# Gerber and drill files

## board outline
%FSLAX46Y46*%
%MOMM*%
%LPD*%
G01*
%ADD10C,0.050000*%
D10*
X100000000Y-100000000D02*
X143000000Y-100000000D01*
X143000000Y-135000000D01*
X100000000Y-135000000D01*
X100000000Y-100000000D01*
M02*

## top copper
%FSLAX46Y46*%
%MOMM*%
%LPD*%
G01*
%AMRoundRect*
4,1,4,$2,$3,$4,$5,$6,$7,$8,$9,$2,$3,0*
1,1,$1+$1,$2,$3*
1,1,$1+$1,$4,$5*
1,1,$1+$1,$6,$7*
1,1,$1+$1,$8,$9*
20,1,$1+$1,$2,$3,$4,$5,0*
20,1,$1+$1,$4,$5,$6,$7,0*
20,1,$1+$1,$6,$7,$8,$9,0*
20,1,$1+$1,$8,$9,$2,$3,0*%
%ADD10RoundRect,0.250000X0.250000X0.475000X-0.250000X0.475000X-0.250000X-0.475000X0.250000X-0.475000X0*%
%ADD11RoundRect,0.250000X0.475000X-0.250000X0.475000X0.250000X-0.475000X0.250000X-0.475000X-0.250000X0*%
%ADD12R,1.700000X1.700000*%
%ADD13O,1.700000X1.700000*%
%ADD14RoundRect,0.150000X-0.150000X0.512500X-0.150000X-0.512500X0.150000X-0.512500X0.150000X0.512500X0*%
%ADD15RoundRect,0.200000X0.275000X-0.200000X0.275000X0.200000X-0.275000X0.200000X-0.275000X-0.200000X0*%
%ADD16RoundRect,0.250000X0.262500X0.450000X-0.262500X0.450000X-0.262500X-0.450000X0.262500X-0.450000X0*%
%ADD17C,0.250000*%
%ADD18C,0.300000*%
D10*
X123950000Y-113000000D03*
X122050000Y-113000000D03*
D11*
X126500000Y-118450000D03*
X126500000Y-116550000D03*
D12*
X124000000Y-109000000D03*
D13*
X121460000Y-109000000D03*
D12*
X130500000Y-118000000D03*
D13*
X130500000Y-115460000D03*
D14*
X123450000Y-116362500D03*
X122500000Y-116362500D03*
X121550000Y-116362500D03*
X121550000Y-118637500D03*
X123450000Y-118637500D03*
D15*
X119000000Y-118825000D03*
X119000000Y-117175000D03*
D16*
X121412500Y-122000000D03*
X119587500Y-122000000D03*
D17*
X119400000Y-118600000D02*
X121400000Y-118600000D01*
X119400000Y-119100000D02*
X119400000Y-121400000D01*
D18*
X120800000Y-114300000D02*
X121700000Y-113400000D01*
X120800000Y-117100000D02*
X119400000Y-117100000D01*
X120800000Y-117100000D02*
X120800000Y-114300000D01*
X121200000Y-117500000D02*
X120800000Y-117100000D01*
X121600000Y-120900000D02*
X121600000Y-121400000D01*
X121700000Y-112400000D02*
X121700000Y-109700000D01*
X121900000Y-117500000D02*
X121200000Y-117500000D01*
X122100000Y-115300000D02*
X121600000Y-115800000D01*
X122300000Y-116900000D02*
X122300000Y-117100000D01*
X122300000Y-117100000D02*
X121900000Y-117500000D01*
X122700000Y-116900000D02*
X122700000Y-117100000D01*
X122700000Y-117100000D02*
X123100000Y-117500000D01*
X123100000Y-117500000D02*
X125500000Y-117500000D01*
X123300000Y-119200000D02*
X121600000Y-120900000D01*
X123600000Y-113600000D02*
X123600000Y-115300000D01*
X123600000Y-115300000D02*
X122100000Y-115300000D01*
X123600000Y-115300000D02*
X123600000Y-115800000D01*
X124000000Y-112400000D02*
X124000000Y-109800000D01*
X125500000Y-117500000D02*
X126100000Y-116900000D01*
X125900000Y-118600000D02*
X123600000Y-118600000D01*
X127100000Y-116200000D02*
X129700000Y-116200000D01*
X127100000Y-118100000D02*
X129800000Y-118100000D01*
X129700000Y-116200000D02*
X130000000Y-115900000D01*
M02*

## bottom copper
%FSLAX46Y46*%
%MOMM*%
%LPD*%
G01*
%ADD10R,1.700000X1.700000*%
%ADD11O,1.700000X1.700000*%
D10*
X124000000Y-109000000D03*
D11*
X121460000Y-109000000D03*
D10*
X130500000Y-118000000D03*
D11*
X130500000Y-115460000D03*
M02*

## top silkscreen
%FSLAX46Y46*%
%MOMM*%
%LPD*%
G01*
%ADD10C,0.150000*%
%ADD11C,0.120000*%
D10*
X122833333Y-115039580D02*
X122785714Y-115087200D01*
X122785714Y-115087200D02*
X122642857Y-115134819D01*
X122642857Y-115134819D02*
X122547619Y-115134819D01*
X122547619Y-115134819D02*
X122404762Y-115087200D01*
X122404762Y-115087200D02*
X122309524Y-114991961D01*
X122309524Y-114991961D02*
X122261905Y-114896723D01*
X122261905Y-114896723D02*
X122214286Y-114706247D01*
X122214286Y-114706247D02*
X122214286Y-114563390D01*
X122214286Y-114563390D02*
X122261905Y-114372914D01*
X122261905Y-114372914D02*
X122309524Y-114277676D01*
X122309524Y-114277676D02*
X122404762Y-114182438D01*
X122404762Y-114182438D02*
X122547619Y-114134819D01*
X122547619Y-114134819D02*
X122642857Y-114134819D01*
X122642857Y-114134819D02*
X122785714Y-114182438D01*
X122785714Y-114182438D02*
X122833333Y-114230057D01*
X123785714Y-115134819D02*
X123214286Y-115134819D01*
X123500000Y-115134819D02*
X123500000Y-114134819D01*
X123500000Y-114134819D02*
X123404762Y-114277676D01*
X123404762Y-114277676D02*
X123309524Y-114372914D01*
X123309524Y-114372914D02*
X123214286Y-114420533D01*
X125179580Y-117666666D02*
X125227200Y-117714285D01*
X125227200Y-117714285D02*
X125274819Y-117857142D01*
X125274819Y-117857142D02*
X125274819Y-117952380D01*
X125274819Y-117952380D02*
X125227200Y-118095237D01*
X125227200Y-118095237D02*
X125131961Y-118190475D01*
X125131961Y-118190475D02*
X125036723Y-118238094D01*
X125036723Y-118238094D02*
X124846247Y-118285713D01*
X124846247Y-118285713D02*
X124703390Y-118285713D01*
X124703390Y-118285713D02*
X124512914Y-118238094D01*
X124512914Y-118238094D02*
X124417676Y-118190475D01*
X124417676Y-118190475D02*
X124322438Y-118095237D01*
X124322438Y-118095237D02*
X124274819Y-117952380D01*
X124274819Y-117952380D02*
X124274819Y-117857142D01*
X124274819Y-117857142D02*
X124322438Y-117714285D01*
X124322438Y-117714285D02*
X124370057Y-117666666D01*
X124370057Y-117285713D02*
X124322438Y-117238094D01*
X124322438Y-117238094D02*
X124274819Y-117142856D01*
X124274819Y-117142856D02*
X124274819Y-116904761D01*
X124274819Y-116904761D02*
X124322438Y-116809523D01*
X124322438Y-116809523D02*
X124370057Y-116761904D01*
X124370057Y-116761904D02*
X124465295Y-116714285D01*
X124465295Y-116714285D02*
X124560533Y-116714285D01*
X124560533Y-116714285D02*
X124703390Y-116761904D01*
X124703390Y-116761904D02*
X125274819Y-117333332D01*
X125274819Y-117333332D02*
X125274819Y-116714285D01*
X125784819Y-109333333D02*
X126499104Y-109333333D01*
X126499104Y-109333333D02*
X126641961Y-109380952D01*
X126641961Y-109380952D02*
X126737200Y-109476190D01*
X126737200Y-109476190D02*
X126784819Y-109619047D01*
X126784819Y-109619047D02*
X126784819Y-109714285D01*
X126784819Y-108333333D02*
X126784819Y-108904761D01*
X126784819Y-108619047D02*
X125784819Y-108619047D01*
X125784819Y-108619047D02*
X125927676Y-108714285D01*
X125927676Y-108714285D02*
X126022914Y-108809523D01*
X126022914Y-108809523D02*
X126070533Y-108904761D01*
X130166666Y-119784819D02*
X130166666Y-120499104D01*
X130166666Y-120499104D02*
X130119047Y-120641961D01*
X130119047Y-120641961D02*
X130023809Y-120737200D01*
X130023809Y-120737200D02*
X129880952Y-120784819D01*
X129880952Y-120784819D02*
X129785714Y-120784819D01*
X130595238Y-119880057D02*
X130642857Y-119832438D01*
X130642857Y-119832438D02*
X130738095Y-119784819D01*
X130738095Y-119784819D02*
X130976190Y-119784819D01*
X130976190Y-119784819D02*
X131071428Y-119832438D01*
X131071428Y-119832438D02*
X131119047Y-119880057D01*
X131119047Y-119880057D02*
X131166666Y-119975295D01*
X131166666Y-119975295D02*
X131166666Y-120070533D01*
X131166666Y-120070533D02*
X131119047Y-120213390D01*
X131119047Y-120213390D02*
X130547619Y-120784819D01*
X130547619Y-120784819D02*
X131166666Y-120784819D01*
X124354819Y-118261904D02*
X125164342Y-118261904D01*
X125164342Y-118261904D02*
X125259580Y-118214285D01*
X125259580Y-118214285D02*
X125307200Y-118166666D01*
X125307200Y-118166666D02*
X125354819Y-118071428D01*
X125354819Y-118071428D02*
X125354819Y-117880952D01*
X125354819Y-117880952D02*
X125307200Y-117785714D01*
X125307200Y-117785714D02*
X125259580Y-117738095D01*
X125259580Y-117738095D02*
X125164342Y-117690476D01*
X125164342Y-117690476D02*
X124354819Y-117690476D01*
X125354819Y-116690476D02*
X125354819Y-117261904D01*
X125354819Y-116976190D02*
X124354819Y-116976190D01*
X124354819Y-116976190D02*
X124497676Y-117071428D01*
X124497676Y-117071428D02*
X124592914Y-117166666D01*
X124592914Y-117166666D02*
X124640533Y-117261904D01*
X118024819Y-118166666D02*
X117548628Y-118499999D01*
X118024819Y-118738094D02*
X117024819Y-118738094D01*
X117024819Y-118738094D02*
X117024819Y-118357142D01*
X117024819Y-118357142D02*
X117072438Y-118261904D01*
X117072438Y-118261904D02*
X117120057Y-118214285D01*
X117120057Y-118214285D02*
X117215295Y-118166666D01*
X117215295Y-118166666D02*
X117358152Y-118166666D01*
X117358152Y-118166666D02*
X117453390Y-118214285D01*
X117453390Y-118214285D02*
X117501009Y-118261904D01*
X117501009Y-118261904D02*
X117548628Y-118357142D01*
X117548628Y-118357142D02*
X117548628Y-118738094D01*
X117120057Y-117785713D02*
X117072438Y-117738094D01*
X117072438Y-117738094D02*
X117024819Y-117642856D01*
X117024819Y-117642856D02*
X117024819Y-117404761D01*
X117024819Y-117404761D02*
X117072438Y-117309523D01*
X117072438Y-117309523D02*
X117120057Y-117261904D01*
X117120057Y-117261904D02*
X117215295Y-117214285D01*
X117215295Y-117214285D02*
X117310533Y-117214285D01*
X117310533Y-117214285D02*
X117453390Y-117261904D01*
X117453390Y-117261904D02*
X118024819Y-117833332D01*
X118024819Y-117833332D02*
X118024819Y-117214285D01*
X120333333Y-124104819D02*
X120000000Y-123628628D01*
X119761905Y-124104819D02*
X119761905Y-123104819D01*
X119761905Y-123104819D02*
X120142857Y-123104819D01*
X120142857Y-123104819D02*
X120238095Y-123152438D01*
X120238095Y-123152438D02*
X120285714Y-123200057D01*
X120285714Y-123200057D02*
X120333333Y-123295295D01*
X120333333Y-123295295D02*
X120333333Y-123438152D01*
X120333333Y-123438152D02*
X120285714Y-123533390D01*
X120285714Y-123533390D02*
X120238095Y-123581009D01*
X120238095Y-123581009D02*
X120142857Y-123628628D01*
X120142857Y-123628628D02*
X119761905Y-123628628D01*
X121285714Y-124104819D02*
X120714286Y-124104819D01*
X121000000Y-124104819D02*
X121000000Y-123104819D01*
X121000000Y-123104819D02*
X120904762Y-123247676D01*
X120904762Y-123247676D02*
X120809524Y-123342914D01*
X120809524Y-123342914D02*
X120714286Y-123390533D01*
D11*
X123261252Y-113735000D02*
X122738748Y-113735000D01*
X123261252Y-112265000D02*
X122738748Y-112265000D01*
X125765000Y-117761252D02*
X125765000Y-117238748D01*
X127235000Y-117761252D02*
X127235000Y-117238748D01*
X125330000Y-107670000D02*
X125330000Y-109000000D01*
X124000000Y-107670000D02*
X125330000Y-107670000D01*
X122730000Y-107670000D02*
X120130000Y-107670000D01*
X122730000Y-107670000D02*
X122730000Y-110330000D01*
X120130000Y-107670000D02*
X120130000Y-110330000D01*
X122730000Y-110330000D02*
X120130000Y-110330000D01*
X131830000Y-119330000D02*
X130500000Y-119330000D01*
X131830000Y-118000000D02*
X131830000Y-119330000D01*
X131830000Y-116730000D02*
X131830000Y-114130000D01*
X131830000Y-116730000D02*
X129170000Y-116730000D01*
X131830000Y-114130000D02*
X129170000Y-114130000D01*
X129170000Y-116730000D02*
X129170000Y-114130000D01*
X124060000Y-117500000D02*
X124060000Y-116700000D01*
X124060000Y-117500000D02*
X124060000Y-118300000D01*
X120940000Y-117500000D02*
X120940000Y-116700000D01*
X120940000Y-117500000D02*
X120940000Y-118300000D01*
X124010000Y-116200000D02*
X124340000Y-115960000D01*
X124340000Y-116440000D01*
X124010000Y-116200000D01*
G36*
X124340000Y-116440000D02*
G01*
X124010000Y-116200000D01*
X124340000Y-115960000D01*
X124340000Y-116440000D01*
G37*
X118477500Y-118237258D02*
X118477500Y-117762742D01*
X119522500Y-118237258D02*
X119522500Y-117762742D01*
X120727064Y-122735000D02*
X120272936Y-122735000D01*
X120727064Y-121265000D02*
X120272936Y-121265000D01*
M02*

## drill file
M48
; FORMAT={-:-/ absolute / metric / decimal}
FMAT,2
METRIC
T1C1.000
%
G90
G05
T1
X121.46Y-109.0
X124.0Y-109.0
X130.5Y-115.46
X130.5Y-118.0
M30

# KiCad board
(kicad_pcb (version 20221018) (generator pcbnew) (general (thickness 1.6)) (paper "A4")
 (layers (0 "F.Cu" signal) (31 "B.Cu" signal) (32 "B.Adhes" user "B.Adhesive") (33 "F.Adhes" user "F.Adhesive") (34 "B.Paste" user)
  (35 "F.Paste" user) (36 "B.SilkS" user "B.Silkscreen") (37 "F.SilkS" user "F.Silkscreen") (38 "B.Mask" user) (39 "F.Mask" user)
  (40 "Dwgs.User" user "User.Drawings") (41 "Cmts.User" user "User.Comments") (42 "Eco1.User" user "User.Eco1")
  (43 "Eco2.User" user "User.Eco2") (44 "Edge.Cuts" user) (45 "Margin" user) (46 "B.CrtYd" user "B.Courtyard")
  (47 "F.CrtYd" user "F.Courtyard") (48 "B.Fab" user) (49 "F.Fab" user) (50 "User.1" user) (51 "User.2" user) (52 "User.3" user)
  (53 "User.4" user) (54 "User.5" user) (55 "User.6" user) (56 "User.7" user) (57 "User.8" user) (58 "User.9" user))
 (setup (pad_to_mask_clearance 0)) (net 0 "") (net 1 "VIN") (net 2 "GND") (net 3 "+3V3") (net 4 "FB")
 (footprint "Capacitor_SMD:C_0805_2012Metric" (layer "F.Cu") (at 123 113 180)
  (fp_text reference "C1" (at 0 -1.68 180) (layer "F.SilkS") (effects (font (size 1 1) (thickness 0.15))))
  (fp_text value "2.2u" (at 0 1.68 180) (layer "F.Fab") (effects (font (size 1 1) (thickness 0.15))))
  (fp_line (start -0.261252 -0.735) (end 0.261252 -0.735) (stroke (width 0.12) (type solid)) (layer "F.SilkS"))
  (fp_line (start -0.261252 0.735) (end 0.261252 0.735) (stroke (width 0.12) (type solid)) (layer "F.SilkS"))
  (pad "1" smd roundrect (at -0.95 0 180) (size 1 1.45) (layers "F.Cu" "F.Paste" "F.Mask") (roundrect_rratio 0.25) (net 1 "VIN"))
  (pad "2" smd roundrect (at 0.95 0 180) (size 1 1.45) (layers "F.Cu" "F.Paste" "F.Mask") (roundrect_rratio 0.25) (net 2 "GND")))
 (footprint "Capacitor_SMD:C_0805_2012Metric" (layer "F.Cu") (at 126.5 117.5 90)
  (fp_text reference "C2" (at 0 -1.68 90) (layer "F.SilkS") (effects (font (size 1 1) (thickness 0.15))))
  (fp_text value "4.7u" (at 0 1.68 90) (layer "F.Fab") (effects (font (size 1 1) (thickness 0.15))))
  (fp_line (start -0.261252 -0.735) (end 0.261252 -0.735) (stroke (width 0.12) (type solid)) (layer "F.SilkS"))
  (fp_line (start -0.261252 0.735) (end 0.261252 0.735) (stroke (width 0.12) (type solid)) (layer "F.SilkS"))
  (pad "1" smd roundrect (at -0.95 0 90) (size 1 1.45) (layers "F.Cu" "F.Paste" "F.Mask") (roundrect_rratio 0.25) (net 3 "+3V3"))
  (pad "2" smd roundrect (at 0.95 0 90) (size 1 1.45) (layers "F.Cu" "F.Paste" "F.Mask") (roundrect_rratio 0.25) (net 2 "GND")))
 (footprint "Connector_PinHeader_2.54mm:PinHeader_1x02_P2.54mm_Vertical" (layer "F.Cu") (at 124 109 -90)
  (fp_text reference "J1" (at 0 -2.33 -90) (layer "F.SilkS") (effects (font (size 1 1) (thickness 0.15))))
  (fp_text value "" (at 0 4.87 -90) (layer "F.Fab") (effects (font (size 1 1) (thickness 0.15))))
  (fp_line (start -1.33 -1.33) (end 0 -1.33) (stroke (width 0.12) (type solid)) (layer "F.SilkS"))
  (fp_line (start -1.33 0) (end -1.33 -1.33) (stroke (width 0.12) (type solid)) (layer "F.SilkS"))
  (fp_line (start -1.33 1.27) (end -1.33 3.87) (stroke (width 0.12) (type solid)) (layer "F.SilkS"))
  (fp_line (start -1.33 1.27) (end 1.33 1.27) (stroke (width 0.12) (type solid)) (layer "F.SilkS"))
  (fp_line (start -1.33 3.87) (end 1.33 3.87) (stroke (width 0.12) (type solid)) (layer "F.SilkS"))
  (fp_line (start 1.33 1.27) (end 1.33 3.87) (stroke (width 0.12) (type solid)) (layer "F.SilkS"))
  (pad "1" thru_hole rect (at 0 0 270) (size 1.7 1.7) (drill 1) (layers "*.Cu" "*.Mask") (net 1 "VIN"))
  (pad "2" thru_hole oval (at 0 2.54 270) (size 1.7 1.7) (drill 1) (layers "*.Cu" "*.Mask") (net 2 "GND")))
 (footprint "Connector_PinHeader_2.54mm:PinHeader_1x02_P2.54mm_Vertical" (layer "F.Cu") (at 130.5 118 180)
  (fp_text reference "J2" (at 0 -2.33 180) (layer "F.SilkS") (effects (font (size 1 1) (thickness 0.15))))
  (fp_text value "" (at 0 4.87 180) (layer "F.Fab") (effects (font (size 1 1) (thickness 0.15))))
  (fp_line (start -1.33 -1.33) (end 0 -1.33) (stroke (width 0.12) (type solid)) (layer "F.SilkS"))
  (fp_line (start -1.33 0) (end -1.33 -1.33) (stroke (width 0.12) (type solid)) (layer "F.SilkS"))
  (fp_line (start -1.33 1.27) (end -1.33 3.87) (stroke (width 0.12) (type solid)) (layer "F.SilkS"))
  (fp_line (start -1.33 1.27) (end 1.33 1.27) (stroke (width 0.12) (type solid)) (layer "F.SilkS"))
  (fp_line (start -1.33 3.87) (end 1.33 3.87) (stroke (width 0.12) (type solid)) (layer "F.SilkS"))
  (fp_line (start 1.33 1.27) (end 1.33 3.87) (stroke (width 0.12) (type solid)) (layer "F.SilkS"))
  (pad "1" thru_hole rect (at 0 0 180) (size 1.7 1.7) (drill 1) (layers "*.Cu" "*.Mask") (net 3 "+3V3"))
  (pad "2" thru_hole oval (at 0 2.54 180) (size 1.7 1.7) (drill 1) (layers "*.Cu" "*.Mask") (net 2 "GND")))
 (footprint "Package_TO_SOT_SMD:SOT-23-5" (layer "F.Cu") (at 122.5 117.5 -90)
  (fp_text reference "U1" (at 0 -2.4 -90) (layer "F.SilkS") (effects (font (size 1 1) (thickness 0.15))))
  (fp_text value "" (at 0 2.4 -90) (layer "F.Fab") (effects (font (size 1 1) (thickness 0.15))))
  (fp_line (start 0 -1.56) (end -0.8 -1.56) (stroke (width 0.12) (type solid)) (layer "F.SilkS"))
  (fp_line (start 0 -1.56) (end 0.8 -1.56) (stroke (width 0.12) (type solid)) (layer "F.SilkS"))
  (fp_line (start 0 1.56) (end -0.8 1.56) (stroke (width 0.12) (type solid)) (layer "F.SilkS"))
  (fp_line (start 0 1.56) (end 0.8 1.56) (stroke (width 0.12) (type solid)) (layer "F.SilkS"))
  (fp_poly
   (pts (xy -1.3 -1.51) (xy -1.54 -1.84) (xy -1.06 -1.84) (xy -1.3 -1.51)) (stroke (width 0.12) (type solid)) (fill solid) (layer "F.SilkS"))
  (pad "1" smd roundrect (at -1.1375 -0.95 270) (size 1.325 0.6) (layers "F.Cu" "F.Paste" "F.Mask") (roundrect_rratio 0.25) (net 1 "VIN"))
  (pad "2" smd roundrect (at -1.1375 0 270) (size 1.325 0.6) (layers "F.Cu" "F.Paste" "F.Mask") (roundrect_rratio 0.25) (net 2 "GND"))
  (pad "3" smd roundrect (at -1.1375 0.95 270) (size 1.325 0.6) (layers "F.Cu" "F.Paste" "F.Mask") (roundrect_rratio 0.25) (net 1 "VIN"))
  (pad "4" smd roundrect (at 1.1375 0.95 270) (size 1.325 0.6) (layers "F.Cu" "F.Paste" "F.Mask") (roundrect_rratio 0.25) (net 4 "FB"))
  (pad "5" smd roundrect (at 1.1375 -0.95 270) (size 1.325 0.6) (layers "F.Cu" "F.Paste" "F.Mask") (roundrect_rratio 0.25) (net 3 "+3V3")))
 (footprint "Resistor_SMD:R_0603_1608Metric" (layer "F.Cu") (at 119 118 90)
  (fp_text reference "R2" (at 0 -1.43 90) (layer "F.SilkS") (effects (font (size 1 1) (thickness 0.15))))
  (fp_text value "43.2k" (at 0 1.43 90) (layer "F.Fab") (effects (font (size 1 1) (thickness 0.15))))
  (fp_line (start -0.237258 -0.5225) (end 0.237258 -0.5225) (stroke (width 0.12) (type solid)) (layer "F.SilkS"))
  (fp_line (start -0.237258 0.5225) (end 0.237258 0.5225) (stroke (width 0.12) (type solid)) (layer "F.SilkS"))
  (pad "1" smd roundrect (at -0.825 0 90) (size 0.8 0.95) (layers "F.Cu" "F.Paste" "F.Mask") (roundrect_rratio 0.25) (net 4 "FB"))
  (pad "2" smd roundrect (at 0.825 0 90) (size 0.8 0.95) (layers "F.Cu" "F.Paste" "F.Mask") (roundrect_rratio 0.25) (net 2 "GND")))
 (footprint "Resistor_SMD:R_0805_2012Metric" (layer "F.Cu") (at 120.5 122 180)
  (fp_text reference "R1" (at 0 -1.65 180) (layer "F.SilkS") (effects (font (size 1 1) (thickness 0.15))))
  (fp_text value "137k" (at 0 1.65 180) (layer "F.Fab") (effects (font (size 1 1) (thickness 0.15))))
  (fp_line (start -0.227064 -0.735) (end 0.227064 -0.735) (stroke (width 0.12) (type solid)) (layer "F.SilkS"))
  (fp_line (start -0.227064 0.735) (end 0.227064 0.735) (stroke (width 0.12) (type solid)) (layer "F.SilkS"))
  (pad "1" smd roundrect (at -0.9125 0 180) (size 1.025 1.4) (layers "F.Cu" "F.Paste" "F.Mask") (roundrect_rratio 0.243902) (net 3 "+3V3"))
  (pad "2" smd roundrect (at 0.9125 0 180) (size 1.025 1.4) (layers "F.Cu" "F.Paste" "F.Mask") (roundrect_rratio 0.243902) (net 4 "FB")))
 (gr_rect (start 100 100) (end 143 135) (stroke (width 0.05) (type default)) (fill none) (layer "Edge.Cuts"))
 (segment (start 119.4 118.6) (end 121.4 118.6) (width 0.25) (layer "F.Cu") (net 4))
 (segment (start 119.4 119.1) (end 119.4 121.4) (width 0.25) (layer "F.Cu") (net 4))
 (segment (start 120.8 114.3) (end 121.7 113.4) (width 0.3) (layer "F.Cu") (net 2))
 (segment (start 120.8 117.1) (end 119.4 117.1) (width 0.3) (layer "F.Cu") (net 2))
 (segment (start 120.8 117.1) (end 120.8 114.3) (width 0.3) (layer "F.Cu") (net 2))
 (segment (start 121.2 117.5) (end 120.8 117.1) (width 0.3) (layer "F.Cu") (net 2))
 (segment (start 121.6 120.9) (end 121.6 121.4) (width 0.3) (layer "F.Cu") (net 3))
 (segment (start 121.7 112.4) (end 121.7 109.7) (width 0.3) (layer "F.Cu") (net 2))
 (segment (start 121.9 117.5) (end 121.2 117.5) (width 0.3) (layer "F.Cu") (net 2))
 (segment (start 122.1 115.3) (end 121.6 115.8) (width 0.3) (layer "F.Cu") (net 1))
 (segment (start 122.3 116.9) (end 122.3 117.1) (width 0.3) (layer "F.Cu") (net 2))
 (segment (start 122.3 117.1) (end 121.9 117.5) (width 0.3) (layer "F.Cu") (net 2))
 (segment (start 122.7 116.9) (end 122.7 117.1) (width 0.3) (layer "F.Cu") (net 2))
 (segment (start 122.7 117.1) (end 123.1 117.5) (width 0.3) (layer "F.Cu") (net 2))
 (segment (start 123.1 117.5) (end 125.5 117.5) (width 0.3) (layer "F.Cu") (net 2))
 (segment (start 123.3 119.2) (end 121.6 120.9) (width 0.3) (layer "F.Cu") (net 3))
 (segment (start 123.6 113.6) (end 123.6 115.3) (width 0.3) (layer "F.Cu") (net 1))
 (segment (start 123.6 115.3) (end 122.1 115.3) (width 0.3) (layer "F.Cu") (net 1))
 (segment (start 123.6 115.3) (end 123.6 115.8) (width 0.3) (layer "F.Cu") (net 1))
 (segment (start 124 112.4) (end 124 109.8) (width 0.3) (layer "F.Cu") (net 1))
 (segment (start 125.5 117.5) (end 126.1 116.9) (width 0.3) (layer "F.Cu") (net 2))
 (segment (start 125.9 118.6) (end 123.6 118.6) (width 0.3) (layer "F.Cu") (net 3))
 (segment (start 127.1 116.2) (end 129.7 116.2) (width 0.3) (layer "F.Cu") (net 2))
 (segment (start 127.1 118.1) (end 129.8 118.1) (width 0.3) (layer "F.Cu") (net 3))
 (segment (start 129.7 116.2) (end 130 115.9) (width 0.3) (layer "F.Cu") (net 2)))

